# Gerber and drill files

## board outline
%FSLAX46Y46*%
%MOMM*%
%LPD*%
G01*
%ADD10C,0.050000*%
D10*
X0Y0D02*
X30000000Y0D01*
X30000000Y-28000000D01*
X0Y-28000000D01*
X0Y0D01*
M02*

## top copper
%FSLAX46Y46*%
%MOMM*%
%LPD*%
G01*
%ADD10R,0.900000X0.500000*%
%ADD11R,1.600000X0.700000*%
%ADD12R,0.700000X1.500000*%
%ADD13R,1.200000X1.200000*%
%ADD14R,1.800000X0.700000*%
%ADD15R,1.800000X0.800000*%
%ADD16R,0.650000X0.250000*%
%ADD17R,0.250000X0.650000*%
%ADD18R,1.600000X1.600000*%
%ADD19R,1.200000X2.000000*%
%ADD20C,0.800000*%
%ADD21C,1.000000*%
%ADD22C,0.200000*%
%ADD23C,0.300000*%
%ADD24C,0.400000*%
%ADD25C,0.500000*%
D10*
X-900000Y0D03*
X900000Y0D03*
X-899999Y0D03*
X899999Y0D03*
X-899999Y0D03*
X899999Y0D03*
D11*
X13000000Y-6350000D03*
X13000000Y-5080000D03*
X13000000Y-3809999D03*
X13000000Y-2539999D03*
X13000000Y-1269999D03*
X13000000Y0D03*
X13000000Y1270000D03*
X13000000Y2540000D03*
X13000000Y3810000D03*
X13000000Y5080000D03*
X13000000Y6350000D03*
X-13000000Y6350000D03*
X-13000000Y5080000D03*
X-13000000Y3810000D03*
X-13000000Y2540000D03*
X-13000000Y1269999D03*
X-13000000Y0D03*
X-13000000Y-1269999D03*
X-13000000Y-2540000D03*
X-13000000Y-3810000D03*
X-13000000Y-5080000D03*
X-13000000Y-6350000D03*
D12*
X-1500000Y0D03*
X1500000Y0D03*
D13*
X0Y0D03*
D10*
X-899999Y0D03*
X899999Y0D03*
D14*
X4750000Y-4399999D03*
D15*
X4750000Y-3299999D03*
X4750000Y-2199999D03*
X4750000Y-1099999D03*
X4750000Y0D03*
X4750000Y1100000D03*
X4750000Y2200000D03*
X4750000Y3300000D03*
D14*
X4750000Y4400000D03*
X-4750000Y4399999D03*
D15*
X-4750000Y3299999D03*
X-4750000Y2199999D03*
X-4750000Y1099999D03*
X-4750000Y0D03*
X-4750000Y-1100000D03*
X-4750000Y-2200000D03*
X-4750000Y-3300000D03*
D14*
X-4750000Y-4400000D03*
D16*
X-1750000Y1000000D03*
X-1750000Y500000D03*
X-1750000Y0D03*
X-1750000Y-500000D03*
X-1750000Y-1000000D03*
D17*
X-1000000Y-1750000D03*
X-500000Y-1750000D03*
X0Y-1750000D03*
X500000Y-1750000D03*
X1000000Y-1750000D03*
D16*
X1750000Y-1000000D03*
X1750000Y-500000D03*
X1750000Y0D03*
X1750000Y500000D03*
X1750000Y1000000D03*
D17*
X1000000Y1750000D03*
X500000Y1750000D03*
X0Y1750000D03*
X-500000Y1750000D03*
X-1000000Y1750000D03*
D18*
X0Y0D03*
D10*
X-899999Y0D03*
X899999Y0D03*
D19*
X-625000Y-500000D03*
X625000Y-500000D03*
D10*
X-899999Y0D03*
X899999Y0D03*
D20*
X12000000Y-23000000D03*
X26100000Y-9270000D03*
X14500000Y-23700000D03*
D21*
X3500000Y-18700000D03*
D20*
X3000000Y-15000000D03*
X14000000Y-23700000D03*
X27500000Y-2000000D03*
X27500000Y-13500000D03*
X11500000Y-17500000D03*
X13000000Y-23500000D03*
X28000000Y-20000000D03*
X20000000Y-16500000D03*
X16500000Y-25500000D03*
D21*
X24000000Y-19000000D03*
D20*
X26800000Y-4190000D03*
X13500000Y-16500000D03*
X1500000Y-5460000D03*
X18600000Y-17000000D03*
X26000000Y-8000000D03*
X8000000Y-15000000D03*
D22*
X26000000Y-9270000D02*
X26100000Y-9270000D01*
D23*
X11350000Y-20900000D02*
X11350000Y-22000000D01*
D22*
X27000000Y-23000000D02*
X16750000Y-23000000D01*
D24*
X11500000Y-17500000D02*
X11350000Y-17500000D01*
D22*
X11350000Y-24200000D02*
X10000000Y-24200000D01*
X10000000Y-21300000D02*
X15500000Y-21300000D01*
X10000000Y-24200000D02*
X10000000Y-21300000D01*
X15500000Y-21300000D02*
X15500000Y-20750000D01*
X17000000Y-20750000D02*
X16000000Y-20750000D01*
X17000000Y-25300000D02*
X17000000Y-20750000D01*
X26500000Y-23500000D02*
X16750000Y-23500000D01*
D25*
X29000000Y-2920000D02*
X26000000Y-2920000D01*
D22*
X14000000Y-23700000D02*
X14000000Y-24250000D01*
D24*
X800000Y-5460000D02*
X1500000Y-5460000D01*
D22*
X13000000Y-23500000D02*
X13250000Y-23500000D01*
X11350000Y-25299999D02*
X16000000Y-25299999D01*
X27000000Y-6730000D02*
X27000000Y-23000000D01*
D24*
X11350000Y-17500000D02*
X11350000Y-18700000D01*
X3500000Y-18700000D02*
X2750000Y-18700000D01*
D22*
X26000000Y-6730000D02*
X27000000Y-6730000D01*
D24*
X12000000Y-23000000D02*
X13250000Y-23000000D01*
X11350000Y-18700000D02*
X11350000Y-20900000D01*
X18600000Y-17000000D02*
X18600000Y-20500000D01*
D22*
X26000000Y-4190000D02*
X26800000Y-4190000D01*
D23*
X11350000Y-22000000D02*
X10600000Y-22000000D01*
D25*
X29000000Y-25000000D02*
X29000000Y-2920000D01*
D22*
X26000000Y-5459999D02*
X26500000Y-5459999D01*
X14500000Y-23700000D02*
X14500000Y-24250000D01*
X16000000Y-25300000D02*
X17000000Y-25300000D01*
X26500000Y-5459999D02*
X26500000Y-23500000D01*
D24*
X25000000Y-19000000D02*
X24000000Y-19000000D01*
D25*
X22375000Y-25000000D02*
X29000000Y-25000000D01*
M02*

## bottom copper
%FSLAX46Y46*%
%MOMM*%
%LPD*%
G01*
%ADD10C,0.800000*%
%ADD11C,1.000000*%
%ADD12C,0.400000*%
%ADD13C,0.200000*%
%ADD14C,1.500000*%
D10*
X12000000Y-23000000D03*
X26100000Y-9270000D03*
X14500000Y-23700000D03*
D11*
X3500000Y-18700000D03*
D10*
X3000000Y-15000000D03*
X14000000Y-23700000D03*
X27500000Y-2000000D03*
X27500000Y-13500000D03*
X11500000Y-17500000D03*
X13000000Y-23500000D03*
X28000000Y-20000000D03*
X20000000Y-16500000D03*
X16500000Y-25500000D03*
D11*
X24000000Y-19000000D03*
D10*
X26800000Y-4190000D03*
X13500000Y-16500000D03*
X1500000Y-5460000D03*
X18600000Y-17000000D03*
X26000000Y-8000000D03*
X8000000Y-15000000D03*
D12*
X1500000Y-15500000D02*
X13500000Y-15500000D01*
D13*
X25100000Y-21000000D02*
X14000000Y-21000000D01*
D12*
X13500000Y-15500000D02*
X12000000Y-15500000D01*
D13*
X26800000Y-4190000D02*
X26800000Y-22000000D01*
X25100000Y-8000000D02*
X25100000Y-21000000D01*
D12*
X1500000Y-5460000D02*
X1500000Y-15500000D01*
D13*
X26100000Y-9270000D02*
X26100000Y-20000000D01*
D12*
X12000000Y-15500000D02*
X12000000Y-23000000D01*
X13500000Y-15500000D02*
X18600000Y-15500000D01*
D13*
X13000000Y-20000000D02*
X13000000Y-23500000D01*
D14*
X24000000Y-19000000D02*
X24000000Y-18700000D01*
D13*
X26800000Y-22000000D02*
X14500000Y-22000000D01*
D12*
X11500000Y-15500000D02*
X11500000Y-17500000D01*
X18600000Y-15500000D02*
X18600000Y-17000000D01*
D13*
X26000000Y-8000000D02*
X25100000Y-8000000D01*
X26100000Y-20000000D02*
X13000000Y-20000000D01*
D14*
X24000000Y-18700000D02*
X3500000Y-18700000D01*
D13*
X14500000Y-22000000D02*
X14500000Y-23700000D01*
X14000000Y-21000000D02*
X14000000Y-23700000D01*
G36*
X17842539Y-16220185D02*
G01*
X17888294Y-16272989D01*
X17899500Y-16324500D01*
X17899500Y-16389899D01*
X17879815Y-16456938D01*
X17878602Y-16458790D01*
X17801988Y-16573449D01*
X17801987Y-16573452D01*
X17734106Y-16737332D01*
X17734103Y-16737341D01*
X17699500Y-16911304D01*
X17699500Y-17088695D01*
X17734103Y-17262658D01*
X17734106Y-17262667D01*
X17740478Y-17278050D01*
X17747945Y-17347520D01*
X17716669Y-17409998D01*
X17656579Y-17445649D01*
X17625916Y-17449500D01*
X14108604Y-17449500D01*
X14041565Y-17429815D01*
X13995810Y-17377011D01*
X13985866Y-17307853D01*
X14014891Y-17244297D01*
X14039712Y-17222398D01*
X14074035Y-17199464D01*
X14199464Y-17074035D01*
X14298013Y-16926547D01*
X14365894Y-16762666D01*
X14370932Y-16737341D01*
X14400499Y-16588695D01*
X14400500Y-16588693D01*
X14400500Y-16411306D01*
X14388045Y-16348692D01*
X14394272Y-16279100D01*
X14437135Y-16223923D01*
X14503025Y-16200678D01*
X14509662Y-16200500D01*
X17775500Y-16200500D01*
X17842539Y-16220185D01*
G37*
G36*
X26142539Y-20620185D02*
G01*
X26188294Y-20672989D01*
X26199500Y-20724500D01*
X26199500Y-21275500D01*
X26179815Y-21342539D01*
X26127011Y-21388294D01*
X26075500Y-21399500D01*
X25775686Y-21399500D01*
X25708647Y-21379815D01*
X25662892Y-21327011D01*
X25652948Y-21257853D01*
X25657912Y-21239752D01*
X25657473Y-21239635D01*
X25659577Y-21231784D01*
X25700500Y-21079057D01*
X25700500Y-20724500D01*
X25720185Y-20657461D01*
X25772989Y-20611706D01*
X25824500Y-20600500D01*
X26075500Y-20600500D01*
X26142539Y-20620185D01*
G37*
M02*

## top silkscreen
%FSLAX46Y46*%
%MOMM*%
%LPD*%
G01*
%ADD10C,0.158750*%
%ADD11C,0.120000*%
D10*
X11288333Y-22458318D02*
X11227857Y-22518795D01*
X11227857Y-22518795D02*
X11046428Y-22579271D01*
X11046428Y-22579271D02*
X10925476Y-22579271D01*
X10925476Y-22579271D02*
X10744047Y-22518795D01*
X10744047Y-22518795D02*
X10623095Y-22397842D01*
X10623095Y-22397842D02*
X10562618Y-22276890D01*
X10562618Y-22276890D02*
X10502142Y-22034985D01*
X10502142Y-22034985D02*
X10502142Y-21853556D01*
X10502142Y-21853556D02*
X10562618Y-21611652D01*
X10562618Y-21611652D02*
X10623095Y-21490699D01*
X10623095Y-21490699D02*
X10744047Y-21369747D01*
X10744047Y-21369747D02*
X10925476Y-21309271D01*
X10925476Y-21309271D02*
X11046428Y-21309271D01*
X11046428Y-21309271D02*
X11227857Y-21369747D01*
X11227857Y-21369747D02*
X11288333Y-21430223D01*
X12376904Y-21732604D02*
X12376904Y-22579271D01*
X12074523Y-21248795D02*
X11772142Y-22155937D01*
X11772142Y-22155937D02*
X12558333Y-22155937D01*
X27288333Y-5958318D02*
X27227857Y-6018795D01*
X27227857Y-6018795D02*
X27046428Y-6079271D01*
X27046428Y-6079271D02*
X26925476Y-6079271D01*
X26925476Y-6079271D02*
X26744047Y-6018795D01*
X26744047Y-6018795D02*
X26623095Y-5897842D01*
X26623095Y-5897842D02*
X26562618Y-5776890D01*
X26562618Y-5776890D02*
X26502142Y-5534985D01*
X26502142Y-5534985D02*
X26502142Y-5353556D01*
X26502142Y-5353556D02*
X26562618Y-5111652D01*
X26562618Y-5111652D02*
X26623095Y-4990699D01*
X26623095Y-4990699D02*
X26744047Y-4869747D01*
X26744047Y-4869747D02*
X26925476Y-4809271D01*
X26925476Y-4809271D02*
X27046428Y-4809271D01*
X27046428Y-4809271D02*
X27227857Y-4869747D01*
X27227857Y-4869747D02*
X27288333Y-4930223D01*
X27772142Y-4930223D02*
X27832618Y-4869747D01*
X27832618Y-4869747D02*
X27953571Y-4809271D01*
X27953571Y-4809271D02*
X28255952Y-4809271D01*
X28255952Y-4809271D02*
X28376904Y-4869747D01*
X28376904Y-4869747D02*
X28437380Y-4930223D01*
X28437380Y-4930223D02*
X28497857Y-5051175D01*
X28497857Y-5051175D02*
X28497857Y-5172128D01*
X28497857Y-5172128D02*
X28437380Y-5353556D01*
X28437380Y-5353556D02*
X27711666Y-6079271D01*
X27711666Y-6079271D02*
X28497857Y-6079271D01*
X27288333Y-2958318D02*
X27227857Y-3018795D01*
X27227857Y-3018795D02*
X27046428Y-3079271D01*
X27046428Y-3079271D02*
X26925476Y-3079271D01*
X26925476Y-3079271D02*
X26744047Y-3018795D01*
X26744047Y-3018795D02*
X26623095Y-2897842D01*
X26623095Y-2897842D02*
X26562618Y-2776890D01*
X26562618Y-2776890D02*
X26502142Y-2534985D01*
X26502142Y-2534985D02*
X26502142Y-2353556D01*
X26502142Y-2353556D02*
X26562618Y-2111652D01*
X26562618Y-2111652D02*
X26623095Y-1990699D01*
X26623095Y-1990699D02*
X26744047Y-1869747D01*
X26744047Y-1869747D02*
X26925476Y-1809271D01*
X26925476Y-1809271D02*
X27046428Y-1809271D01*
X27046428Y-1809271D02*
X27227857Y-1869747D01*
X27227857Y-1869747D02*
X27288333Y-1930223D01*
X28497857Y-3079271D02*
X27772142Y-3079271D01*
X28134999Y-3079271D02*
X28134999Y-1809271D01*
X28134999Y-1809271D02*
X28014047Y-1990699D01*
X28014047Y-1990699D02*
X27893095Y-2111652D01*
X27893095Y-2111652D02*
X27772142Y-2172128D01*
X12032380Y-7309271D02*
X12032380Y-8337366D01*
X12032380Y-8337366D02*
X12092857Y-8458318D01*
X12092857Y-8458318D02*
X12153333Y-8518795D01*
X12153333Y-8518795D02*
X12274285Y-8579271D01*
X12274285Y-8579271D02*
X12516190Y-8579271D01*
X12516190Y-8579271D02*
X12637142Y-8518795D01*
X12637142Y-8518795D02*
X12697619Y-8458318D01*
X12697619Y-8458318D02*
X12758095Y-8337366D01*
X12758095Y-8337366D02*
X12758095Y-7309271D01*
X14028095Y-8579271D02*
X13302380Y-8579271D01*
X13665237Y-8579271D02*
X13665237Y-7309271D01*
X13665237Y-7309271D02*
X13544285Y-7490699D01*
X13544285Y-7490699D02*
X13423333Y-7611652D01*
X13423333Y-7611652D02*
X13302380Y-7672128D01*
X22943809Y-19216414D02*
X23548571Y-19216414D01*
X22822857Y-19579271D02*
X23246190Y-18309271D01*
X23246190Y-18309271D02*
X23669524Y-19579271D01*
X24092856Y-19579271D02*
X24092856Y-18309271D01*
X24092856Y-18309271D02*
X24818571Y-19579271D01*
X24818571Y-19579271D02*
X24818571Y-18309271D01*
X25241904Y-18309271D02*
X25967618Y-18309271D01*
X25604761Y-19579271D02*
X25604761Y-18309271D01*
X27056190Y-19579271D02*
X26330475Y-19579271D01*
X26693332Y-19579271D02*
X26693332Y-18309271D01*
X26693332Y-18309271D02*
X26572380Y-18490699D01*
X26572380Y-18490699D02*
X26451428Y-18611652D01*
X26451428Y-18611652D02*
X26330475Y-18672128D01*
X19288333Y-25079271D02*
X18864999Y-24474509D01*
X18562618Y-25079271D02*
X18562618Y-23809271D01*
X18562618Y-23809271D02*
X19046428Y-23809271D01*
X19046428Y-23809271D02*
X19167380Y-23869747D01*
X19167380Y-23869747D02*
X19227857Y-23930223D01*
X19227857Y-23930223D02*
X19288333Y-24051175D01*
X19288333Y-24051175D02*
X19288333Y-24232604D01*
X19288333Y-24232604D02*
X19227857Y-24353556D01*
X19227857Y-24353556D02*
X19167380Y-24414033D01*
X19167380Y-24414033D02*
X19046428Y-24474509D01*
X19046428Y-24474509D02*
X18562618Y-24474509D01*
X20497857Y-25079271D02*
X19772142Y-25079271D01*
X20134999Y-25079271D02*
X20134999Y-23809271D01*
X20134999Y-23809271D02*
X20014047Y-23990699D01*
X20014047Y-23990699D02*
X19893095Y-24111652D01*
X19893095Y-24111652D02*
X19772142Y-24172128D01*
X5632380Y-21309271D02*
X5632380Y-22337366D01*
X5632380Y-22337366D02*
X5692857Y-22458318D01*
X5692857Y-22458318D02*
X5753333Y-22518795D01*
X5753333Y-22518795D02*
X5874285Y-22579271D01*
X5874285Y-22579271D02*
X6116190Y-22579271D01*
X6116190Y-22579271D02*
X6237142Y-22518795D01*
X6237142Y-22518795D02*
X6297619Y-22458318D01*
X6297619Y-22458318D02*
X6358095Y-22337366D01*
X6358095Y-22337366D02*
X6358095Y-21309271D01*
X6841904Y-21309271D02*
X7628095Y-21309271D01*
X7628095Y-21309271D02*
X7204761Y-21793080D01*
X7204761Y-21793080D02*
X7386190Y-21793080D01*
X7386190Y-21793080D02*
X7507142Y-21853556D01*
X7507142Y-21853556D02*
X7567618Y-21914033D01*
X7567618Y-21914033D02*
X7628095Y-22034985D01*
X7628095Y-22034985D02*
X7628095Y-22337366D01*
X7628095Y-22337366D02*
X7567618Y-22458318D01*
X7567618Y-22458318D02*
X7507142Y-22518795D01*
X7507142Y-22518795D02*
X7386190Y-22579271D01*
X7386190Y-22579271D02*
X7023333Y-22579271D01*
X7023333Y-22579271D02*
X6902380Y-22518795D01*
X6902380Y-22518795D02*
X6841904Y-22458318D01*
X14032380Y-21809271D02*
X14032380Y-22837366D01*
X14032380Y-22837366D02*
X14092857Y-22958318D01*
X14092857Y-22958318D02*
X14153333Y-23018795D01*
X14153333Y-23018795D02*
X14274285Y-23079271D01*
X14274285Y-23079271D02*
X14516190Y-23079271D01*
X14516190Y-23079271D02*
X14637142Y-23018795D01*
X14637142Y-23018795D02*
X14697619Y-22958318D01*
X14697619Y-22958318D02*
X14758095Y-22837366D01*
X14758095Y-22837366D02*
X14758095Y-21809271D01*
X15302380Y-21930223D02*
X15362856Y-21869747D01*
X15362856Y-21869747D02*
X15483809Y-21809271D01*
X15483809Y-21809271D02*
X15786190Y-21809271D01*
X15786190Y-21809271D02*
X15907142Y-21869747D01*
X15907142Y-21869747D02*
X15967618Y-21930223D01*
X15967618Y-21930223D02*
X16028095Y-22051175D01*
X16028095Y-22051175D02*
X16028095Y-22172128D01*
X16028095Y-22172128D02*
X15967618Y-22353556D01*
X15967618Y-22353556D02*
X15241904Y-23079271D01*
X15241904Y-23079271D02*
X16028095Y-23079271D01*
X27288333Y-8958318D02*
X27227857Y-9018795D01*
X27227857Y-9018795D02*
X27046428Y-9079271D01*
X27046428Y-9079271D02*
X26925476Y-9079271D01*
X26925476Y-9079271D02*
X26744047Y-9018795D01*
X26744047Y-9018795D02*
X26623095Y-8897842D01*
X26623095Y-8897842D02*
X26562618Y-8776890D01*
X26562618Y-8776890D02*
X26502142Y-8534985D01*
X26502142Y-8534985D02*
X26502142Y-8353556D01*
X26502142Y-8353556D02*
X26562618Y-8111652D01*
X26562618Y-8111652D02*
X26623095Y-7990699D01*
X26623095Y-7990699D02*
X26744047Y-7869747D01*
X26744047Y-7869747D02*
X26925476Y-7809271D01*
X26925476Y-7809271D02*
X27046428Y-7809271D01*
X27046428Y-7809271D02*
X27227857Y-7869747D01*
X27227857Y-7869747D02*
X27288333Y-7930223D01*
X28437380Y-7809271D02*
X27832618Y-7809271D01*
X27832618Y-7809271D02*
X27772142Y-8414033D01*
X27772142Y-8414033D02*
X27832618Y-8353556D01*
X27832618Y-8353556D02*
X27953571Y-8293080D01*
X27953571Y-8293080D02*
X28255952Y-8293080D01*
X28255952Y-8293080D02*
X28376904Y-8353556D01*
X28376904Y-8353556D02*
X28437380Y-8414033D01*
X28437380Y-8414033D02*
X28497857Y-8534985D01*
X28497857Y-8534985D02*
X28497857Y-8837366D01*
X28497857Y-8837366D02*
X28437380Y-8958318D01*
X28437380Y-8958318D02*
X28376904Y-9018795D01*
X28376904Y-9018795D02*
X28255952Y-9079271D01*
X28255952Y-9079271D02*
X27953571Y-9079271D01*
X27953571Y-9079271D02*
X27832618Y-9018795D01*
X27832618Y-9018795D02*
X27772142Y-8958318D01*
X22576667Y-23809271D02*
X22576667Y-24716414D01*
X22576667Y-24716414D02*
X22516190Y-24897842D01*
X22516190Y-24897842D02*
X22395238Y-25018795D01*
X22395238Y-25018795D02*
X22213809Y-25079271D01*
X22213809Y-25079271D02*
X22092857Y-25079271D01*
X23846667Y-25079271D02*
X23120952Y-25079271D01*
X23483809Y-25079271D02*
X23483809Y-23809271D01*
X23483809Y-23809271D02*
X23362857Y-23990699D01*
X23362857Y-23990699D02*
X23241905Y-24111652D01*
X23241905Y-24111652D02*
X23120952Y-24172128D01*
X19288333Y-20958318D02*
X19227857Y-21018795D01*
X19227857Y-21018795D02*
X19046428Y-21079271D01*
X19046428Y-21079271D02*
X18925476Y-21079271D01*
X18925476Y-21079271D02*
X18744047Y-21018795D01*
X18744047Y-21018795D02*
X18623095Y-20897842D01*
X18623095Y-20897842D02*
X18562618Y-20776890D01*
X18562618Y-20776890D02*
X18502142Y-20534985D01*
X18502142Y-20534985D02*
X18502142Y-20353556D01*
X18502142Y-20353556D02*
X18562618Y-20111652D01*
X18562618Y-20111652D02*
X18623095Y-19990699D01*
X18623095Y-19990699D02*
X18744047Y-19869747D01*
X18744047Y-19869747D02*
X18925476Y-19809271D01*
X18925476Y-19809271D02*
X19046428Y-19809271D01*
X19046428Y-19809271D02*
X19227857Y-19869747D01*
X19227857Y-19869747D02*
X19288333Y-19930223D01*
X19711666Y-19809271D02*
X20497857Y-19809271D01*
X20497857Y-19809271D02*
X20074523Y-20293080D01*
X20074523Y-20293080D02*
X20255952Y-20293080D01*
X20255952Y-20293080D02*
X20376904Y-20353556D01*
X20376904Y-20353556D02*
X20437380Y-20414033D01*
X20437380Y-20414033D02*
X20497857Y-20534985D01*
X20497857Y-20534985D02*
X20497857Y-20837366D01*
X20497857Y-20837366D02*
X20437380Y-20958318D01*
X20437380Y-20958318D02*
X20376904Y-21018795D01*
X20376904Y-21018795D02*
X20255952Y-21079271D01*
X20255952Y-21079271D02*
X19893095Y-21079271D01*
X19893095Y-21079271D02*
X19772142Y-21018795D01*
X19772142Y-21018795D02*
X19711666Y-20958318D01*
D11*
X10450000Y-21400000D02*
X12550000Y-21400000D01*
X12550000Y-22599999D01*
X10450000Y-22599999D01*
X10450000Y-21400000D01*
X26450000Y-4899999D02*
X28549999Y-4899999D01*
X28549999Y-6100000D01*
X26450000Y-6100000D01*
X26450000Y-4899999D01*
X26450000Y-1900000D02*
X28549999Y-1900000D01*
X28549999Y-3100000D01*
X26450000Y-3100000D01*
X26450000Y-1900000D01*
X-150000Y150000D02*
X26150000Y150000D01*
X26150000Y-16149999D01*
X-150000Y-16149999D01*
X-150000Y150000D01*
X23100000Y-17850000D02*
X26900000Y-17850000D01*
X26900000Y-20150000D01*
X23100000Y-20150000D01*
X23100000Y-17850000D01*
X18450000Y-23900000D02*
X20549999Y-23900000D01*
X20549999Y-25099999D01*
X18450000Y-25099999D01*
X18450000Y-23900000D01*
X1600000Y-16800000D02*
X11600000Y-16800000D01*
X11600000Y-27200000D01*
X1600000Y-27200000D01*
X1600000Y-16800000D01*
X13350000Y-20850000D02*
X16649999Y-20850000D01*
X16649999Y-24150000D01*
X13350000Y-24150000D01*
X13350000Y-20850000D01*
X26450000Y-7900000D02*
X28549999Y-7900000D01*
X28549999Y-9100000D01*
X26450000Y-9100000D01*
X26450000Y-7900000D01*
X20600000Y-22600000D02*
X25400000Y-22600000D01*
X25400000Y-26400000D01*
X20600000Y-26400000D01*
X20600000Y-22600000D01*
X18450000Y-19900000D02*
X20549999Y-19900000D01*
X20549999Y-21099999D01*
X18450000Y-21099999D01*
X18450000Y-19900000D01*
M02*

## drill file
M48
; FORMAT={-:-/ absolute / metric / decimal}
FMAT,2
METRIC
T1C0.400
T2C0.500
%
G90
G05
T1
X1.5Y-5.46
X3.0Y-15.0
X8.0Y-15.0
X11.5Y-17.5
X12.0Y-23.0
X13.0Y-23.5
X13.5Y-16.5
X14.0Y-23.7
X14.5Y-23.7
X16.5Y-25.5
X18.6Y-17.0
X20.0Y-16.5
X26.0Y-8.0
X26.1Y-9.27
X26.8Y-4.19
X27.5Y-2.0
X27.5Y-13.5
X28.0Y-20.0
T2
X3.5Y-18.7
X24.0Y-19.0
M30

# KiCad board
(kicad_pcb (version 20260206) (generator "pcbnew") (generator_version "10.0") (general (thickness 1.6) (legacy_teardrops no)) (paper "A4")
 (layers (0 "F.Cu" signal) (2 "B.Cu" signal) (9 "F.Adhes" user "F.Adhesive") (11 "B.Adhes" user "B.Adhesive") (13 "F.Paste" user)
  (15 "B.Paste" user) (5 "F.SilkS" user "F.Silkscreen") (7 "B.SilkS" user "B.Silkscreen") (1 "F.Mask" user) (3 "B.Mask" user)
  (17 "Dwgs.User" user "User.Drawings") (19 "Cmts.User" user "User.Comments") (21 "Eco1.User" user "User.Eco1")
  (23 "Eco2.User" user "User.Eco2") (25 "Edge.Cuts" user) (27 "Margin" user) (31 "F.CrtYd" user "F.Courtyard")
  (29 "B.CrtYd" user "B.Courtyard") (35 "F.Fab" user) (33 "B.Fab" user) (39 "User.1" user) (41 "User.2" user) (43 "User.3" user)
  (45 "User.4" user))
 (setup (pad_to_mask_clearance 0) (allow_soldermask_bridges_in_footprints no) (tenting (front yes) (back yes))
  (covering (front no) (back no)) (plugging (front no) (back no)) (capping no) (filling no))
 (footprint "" (layer "F.Cu") (at 11.5 22)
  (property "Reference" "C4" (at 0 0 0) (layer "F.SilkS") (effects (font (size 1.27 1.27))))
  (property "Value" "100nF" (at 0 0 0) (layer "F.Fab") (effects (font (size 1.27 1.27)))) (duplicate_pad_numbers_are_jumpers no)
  (fp_rect (start -1.05 -0.6) (end 1.05 0.599999) (stroke (width 0.12) (type default)) (fill no) (layer "F.SilkS"))
  (pad "1" smd rect (at -12.4 -22) (size 0.9 0.5) (layers "F.Cu" "F.Mask" "F.Paste") (thermal_bridge_angle 45))
  (pad "2" smd rect (at -10.6 -22) (size 0.9 0.5) (layers "F.Cu" "F.Mask" "F.Paste") (thermal_bridge_angle 45)))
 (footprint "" (layer "F.Cu") (at 27.5 5.5)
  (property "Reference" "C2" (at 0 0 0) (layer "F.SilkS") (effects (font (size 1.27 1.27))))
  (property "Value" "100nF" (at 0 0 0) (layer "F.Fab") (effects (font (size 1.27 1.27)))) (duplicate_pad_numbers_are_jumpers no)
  (fp_rect (start -1.05 -0.600001) (end 1.049999 0.6) (stroke (width 0.12) (type default)) (fill no) (layer "F.SilkS"))
  (pad "1" smd rect (at -28.399999 -5.5) (size 0.9 0.5) (layers "F.Cu" "F.Mask" "F.Paste") (thermal_bridge_angle 45))
  (pad "2" smd rect (at -26.600001 -5.5) (size 0.9 0.5) (layers "F.Cu" "F.Mask" "F.Paste") (thermal_bridge_angle 45)))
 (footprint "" (layer "F.Cu") (at 27.5 2.5)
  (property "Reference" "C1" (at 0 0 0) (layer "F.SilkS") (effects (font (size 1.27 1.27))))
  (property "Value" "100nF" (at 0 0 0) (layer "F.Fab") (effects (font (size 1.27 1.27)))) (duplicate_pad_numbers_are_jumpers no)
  (fp_rect (start -1.05 -0.6) (end 1.049999 0.6) (stroke (width 0.12) (type default)) (fill no) (layer "F.SilkS"))
  (pad "1" smd rect (at -28.399999 -2.5) (size 0.9 0.5) (layers "F.Cu" "F.Mask" "F.Paste") (thermal_bridge_angle 45))
  (pad "2" smd rect (at -26.600001 -2.5) (size 0.9 0.5) (layers "F.Cu" "F.Mask" "F.Paste") (thermal_bridge_angle 45)))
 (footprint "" (layer "F.Cu") (at 13 8)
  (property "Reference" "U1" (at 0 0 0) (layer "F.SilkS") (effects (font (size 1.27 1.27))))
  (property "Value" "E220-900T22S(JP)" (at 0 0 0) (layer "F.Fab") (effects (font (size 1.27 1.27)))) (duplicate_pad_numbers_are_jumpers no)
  (fp_rect (start -13.15 -8.15) (end 13.15 8.149999) (stroke (width 0.12) (type default)) (fill no) (layer "F.SilkS"))
  (pad "1" smd rect (at 0 -1.65) (size 1.6 0.7) (layers "F.Cu" "F.Mask" "F.Paste") (thermal_bridge_angle 45))
  (pad "2" smd rect (at 0 -2.92) (size 1.6 0.7) (layers "F.Cu" "F.Mask" "F.Paste") (thermal_bridge_angle 45))
  (pad "3" smd rect (at 0 -4.190001) (size 1.6 0.7) (layers "F.Cu" "F.Mask" "F.Paste") (thermal_bridge_angle 45))
  (pad "4" smd rect (at 0 -5.460001) (size 1.6 0.7) (layers "F.Cu" "F.Mask" "F.Paste") (thermal_bridge_angle 45))
  (pad "5" smd rect (at 0 -6.730001) (size 1.6 0.7) (layers "F.Cu" "F.Mask" "F.Paste") (thermal_bridge_angle 45))
  (pad "6" smd rect (at 0 -8) (size 1.6 0.7) (layers "F.Cu" "F.Mask" "F.Paste") (thermal_bridge_angle 45))
  (pad "7" smd rect (at 0 -9.27) (size 1.6 0.7) (layers "F.Cu" "F.Mask" "F.Paste") (thermal_bridge_angle 45))
  (pad "8" smd rect (at 0 -10.54) (size 1.6 0.7) (layers "F.Cu" "F.Mask" "F.Paste") (thermal_bridge_angle 45))
  (pad "9" smd rect (at 0 -11.81) (size 1.6 0.7) (layers "F.Cu" "F.Mask" "F.Paste") (thermal_bridge_angle 45))
  (pad "10" smd rect (at 0 -13.08) (size 1.6 0.7) (layers "F.Cu" "F.Mask" "F.Paste") (thermal_bridge_angle 45))
  (pad "11" smd rect (at 0 -14.35) (size 1.6 0.7) (layers "F.Cu" "F.Mask" "F.Paste") (thermal_bridge_angle 45))
  (pad "12" smd rect (at -26 -14.35) (size 1.6 0.7) (layers "F.Cu" "F.Mask" "F.Paste") (thermal_bridge_angle 45))
  (pad "13" smd rect (at -26 -13.08) (size 1.6 0.7) (layers "F.Cu" "F.Mask" "F.Paste") (thermal_bridge_angle 45))
  (pad "14" smd rect (at -26 -11.81) (size 1.6 0.7) (layers "F.Cu" "F.Mask" "F.Paste") (thermal_bridge_angle 45))
  (pad "15" smd rect (at -26 -10.54) (size 1.6 0.7) (layers "F.Cu" "F.Mask" "F.Paste") (thermal_bridge_angle 45))
  (pad "16" smd rect (at -26 -9.269999) (size 1.6 0.7) (layers "F.Cu" "F.Mask" "F.Paste") (thermal_bridge_angle 45))
  (pad "17" smd rect (at -26 -8) (size 1.6 0.7) (layers "F.Cu" "F.Mask" "F.Paste") (thermal_bridge_angle 45))
  (pad "18" smd rect (at -26 -6.730001) (size 1.6 0.7) (layers "F.Cu" "F.Mask" "F.Paste") (thermal_bridge_angle 45))
  (pad "19" smd rect (at -26 -5.46) (size 1.6 0.7) (layers "F.Cu" "F.Mask" "F.Paste") (thermal_bridge_angle 45))
  (pad "20" smd rect (at -26 -4.19) (size 1.6 0.7) (layers "F.Cu" "F.Mask" "F.Paste") (thermal_bridge_angle 45))
  (pad "21" smd rect (at -26 -2.92) (size 1.6 0.7) (layers "F.Cu" "F.Mask" "F.Paste") (thermal_bridge_angle 45))
  (pad "22" smd rect (at -26 -1.65) (size 1.6 0.7) (layers "F.Cu" "F.Mask" "F.Paste") (thermal_bridge_angle 45)))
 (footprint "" (layer "F.Cu") (at 25 19)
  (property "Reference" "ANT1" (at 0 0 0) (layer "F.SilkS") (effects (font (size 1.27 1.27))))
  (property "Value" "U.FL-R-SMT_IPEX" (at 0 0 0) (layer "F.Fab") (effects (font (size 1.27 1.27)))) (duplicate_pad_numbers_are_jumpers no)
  (fp_rect (start -1.9 -1.15) (end 1.9 1.15) (stroke (width 0.12) (type default)) (fill no) (layer "F.SilkS"))
  (pad "G1" smd rect (at -26.5 -19) (size 0.7 1.5) (layers "F.Cu" "F.Mask" "F.Paste") (thermal_bridge_angle 45))
  (pad "G2" smd rect (at -23.5 -19) (size 0.7 1.5) (layers "F.Cu" "F.Mask" "F.Paste") (thermal_bridge_angle 45))
  (pad "S" smd rect (at -25 -19) (size 1.2 1.2) (layers "F.Cu" "F.Mask" "F.Paste") (thermal_bridge_angle 45)))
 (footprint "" (layer "F.Cu") (at 19.5 24.5)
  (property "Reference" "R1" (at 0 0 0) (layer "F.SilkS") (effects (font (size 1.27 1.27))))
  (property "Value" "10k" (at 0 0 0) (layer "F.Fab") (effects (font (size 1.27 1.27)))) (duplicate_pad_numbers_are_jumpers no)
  (fp_rect (start -1.05 -0.6) (end 1.049999 0.599999) (stroke (width 0.12) (type default)) (fill no) (layer "F.SilkS"))
  (pad "1" smd rect (at -20.399999 -24.5) (size 0.9 0.5) (layers "F.Cu" "F.Mask" "F.Paste") (thermal_bridge_angle 45))
  (pad "2" smd rect (at -18.600001 -24.5) (size 0.9 0.5) (layers "F.Cu" "F.Mask" "F.Paste") (thermal_bridge_angle 45)))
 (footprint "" (layer "F.Cu") (at 6.6 22)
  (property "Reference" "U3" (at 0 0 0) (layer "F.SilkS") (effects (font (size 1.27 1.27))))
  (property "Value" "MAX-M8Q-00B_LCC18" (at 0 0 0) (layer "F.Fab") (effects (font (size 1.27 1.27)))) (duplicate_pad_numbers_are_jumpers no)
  (fp_rect (start -5 -5.2) (end 5 5.2) (stroke (width 0.12) (type default)) (fill no) (layer "F.SilkS"))
  (pad "1" smd rect (at -1.85 -17.600001) (size 1.8 0.7) (layers "F.Cu" "F.Mask" "F.Paste") (thermal_bridge_angle 45))
  (pad "2" smd rect (at -1.85 -18.700001) (size 1.8 0.8) (layers "F.Cu" "F.Mask" "F.Paste") (thermal_bridge_angle 45))
  (pad "3" smd rect (at -1.85 -19.800001) (size 1.8 0.8) (layers "F.Cu" "F.Mask" "F.Paste") (thermal_bridge_angle 45))
  (pad "4" smd rect (at -1.85 -20.900001) (size 1.8 0.8) (layers "F.Cu" "F.Mask" "F.Paste") (thermal_bridge_angle 45))
  (pad "5" smd rect (at -1.85 -22) (size 1.8 0.8) (layers "F.Cu" "F.Mask" "F.Paste") (thermal_bridge_angle 45))
  (pad "6" smd rect (at -1.85 -23.1) (size 1.8 0.8) (layers "F.Cu" "F.Mask" "F.Paste") (thermal_bridge_angle 45))
  (pad "7" smd rect (at -1.85 -24.2) (size 1.8 0.8) (layers "F.Cu" "F.Mask" "F.Paste") (thermal_bridge_angle 45))
  (pad "8" smd rect (at -1.85 -25.3) (size 1.8 0.8) (layers "F.Cu" "F.Mask" "F.Paste") (thermal_bridge_angle 45))
  (pad "9" smd rect (at -1.85 -26.4) (size 1.8 0.7) (layers "F.Cu" "F.Mask" "F.Paste") (thermal_bridge_angle 45))
  (pad "10" smd rect (at -11.35 -26.399999) (size 1.8 0.7) (layers "F.Cu" "F.Mask" "F.Paste") (thermal_bridge_angle 45))
  (pad "11" smd rect (at -11.35 -25.299999) (size 1.8 0.8) (layers "F.Cu" "F.Mask" "F.Paste") (thermal_bridge_angle 45))
  (pad "12" smd rect (at -11.35 -24.199999) (size 1.8 0.8) (layers "F.Cu" "F.Mask" "F.Paste") (thermal_bridge_angle 45))
  (pad "13" smd rect (at -11.35 -23.099999) (size 1.8 0.8) (layers "F.Cu" "F.Mask" "F.Paste") (thermal_bridge_angle 45))
  (pad "14" smd rect (at -11.35 -22) (size 1.8 0.8) (layers "F.Cu" "F.Mask" "F.Paste") (thermal_bridge_angle 45))
  (pad "15" smd rect (at -11.35 -20.9) (size 1.8 0.8) (layers "F.Cu" "F.Mask" "F.Paste") (thermal_bridge_angle 45))
  (pad "16" smd rect (at -11.35 -19.8) (size 1.8 0.8) (layers "F.Cu" "F.Mask" "F.Paste") (thermal_bridge_angle 45))
  (pad "17" smd rect (at -11.35 -18.7) (size 1.8 0.8) (layers "F.Cu" "F.Mask" "F.Paste") (thermal_bridge_angle 45))
  (pad "18" smd rect (at -11.35 -17.6) (size 1.8 0.7) (layers "F.Cu" "F.Mask" "F.Paste") (thermal_bridge_angle 45)))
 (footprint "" (layer "F.Cu") (at 15 22.5)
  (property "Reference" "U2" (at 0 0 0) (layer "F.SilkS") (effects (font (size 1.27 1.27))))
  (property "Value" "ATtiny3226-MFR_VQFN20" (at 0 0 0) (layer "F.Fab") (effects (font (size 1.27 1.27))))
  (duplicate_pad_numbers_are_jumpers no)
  (fp_rect (start -1.65 -1.65) (end 1.649999 1.65) (stroke (width 0.12) (type default)) (fill no) (layer "F.SilkS"))
  (pad "1" smd rect (at -16.75 -23.5) (size 0.65 0.25) (layers "F.Cu" "F.Mask" "F.Paste") (thermal_bridge_angle 45))
  (pad "2" smd rect (at -16.75 -23) (size 0.65 0.25) (layers "F.Cu" "F.Mask" "F.Paste") (thermal_bridge_angle 45))
  (pad "3" smd rect (at -16.75 -22.5) (size 0.65 0.25) (layers "F.Cu" "F.Mask" "F.Paste") (thermal_bridge_angle 45))
  (pad "4" smd rect (at -16.75 -22) (size 0.65 0.25) (layers "F.Cu" "F.Mask" "F.Paste") (thermal_bridge_angle 45))
  (pad "5" smd rect (at -16.75 -21.5) (size 0.65 0.25) (layers "F.Cu" "F.Mask" "F.Paste") (thermal_bridge_angle 45))
  (pad "6" smd rect (at -16 -20.75) (size 0.25 0.65) (layers "F.Cu" "F.Mask" "F.Paste") (thermal_bridge_angle 45))
  (pad "7" smd rect (at -15.5 -20.75) (size 0.25 0.65) (layers "F.Cu" "F.Mask" "F.Paste") (thermal_bridge_angle 45))
  (pad "8" smd rect (at -15 -20.75) (size 0.25 0.65) (layers "F.Cu" "F.Mask" "F.Paste") (thermal_bridge_angle 45))
  (pad "9" smd rect (at -14.5 -20.75) (size 0.25 0.65) (layers "F.Cu" "F.Mask" "F.Paste") (thermal_bridge_angle 45))
  (pad "10" smd rect (at -14 -20.75) (size 0.25 0.65) (layers "F.Cu" "F.Mask" "F.Paste") (thermal_bridge_angle 45))
  (pad "11" smd rect (at -13.25 -21.5) (size 0.65 0.25) (layers "F.Cu" "F.Mask" "F.Paste") (thermal_bridge_angle 45))
  (pad "12" smd rect (at -13.25 -22) (size 0.65 0.25) (layers "F.Cu" "F.Mask" "F.Paste") (thermal_bridge_angle 45))
  (pad "13" smd rect (at -13.25 -22.5) (size 0.65 0.25) (layers "F.Cu" "F.Mask" "F.Paste") (thermal_bridge_angle 45))
  (pad "14" smd rect (at -13.25 -23) (size 0.65 0.25) (layers "F.Cu" "F.Mask" "F.Paste") (thermal_bridge_angle 45))
  (pad "15" smd rect (at -13.25 -23.5) (size 0.65 0.25) (layers "F.Cu" "F.Mask" "F.Paste") (thermal_bridge_angle 45))
  (pad "16" smd rect (at -14 -24.25) (size 0.25 0.65) (layers "F.Cu" "F.Mask" "F.Paste") (thermal_bridge_angle 45))
  (pad "17" smd rect (at -14.5 -24.25) (size 0.25 0.65) (layers "F.Cu" "F.Mask" "F.Paste") (thermal_bridge_angle 45))
  (pad "18" smd rect (at -15 -24.25) (size 0.25 0.65) (layers "F.Cu" "F.Mask" "F.Paste") (thermal_bridge_angle 45))
  (pad "19" smd rect (at -15.5 -24.25) (size 0.25 0.65) (layers "F.Cu" "F.Mask" "F.Paste") (thermal_bridge_angle 45))
  (pad "20" smd rect (at -16 -24.25) (size 0.25 0.65) (layers "F.Cu" "F.Mask" "F.Paste") (thermal_bridge_angle 45))
  (pad "EP" smd rect (at -15 -22.5) (size 1.6 1.6) (layers "F.Cu" "F.Mask" "F.Paste") (thermal_bridge_angle 45)))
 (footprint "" (layer "F.Cu") (at 27.5 8.5)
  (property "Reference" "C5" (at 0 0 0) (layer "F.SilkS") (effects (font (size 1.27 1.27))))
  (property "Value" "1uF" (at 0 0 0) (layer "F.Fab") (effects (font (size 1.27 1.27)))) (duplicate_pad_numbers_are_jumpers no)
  (fp_rect (start -1.05 -0.6) (end 1.049999 0.6) (stroke (width 0.12) (type default)) (fill no) (layer "F.SilkS"))
  (pad "1" smd rect (at -28.399999 -8.5) (size 0.9 0.5) (layers "F.Cu" "F.Mask" "F.Paste") (thermal_bridge_angle 45))
  (pad "2" smd rect (at -26.600001 -8.5) (size 0.9 0.5) (layers "F.Cu" "F.Mask" "F.Paste") (thermal_bridge_angle 45)))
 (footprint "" (layer "F.Cu") (at 23 24.5)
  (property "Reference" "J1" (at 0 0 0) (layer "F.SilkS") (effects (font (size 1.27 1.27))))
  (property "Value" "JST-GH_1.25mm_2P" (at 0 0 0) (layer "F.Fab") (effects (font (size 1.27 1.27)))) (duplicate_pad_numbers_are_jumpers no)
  (fp_rect (start -2.4 -1.9) (end 2.4 1.9) (stroke (width 0.12) (type default)) (fill no) (layer "F.SilkS"))
  (pad "1" smd rect (at -23.625 -24) (size 1.2 2) (layers "F.Cu" "F.Mask" "F.Paste") (thermal_bridge_angle 45))
  (pad "2" smd rect (at -22.375 -24) (size 1.2 2) (layers "F.Cu" "F.Mask" "F.Paste") (thermal_bridge_angle 45)))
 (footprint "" (layer "F.Cu") (at 19.5 20.5)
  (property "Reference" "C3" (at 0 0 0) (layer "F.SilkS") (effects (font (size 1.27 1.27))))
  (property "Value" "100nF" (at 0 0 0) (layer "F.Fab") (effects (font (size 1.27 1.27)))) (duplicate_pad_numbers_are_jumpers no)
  (fp_rect (start -1.05 -0.6) (end 1.049999 0.599999) (stroke (width 0.12) (type default)) (fill no) (layer "F.SilkS"))
  (pad "1" smd rect (at -20.399999 -20.5) (size 0.9 0.5) (layers "F.Cu" "F.Mask" "F.Paste") (thermal_bridge_angle 45))
  (pad "2" smd rect (at -18.600001 -20.5) (size 0.9 0.5) (layers "F.Cu" "F.Mask" "F.Paste") (thermal_bridge_angle 45)))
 (gr_rect (start 0 0) (end 30 28) (stroke (width 0.05) (type default)) (fill no) (layer "Edge.Cuts"))
 (segment (start 26 9.27) (end 26.1 9.27) (width 0.2) (layer "F.Cu") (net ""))
 (segment (start 11.35 20.9) (end 11.35 22) (width 0.3) (layer "F.Cu") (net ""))
 (segment (start 27 23) (end 16.75 23) (width 0.2) (layer "F.Cu") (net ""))
 (segment (start 11.5 17.5) (end 11.35 17.5) (width 0.4) (layer "F.Cu") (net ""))
 (segment (start 11.35 24.2) (end 10 24.2) (width 0.2) (layer "F.Cu") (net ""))
 (segment (start 10 21.3) (end 15.5 21.3) (width 0.2) (layer "F.Cu") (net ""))
 (segment (start 10 24.2) (end 10 21.3) (width 0.2) (layer "F.Cu") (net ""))
 (segment (start 15.5 21.3) (end 15.5 20.75) (width 0.2) (layer "F.Cu") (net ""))
 (segment (start 17 20.75) (end 16 20.75) (width 0.2) (layer "F.Cu") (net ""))
 (segment (start 17 25.3) (end 17 20.75) (width 0.2) (layer "F.Cu") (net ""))
 (segment (start 26.5 23.5) (end 16.75 23.5) (width 0.2) (layer "F.Cu") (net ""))
 (segment (start 29 2.92) (end 26 2.92) (width 0.5) (layer "F.Cu") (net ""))
 (segment (start 14 23.7) (end 14 24.25) (width 0.2) (layer "F.Cu") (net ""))
 (segment (start 0.8 5.46) (end 1.5 5.46) (width 0.4) (layer "F.Cu") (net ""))
 (segment (start 13 23.5) (end 13.25 23.5) (width 0.2) (layer "F.Cu") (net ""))
 (segment (start 11.35 25.299999) (end 16 25.299999) (width 0.2) (layer "F.Cu") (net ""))
 (segment (start 27 6.73) (end 27 23) (width 0.2) (layer "F.Cu") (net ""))
 (segment (start 11.35 17.5) (end 11.35 18.7) (width 0.4) (layer "F.Cu") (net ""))
 (segment (start 3.5 18.7) (end 2.75 18.7) (width 0.4) (layer "F.Cu") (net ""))
 (segment (start 26 6.73) (end 27 6.73) (width 0.2) (layer "F.Cu") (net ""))
 (segment (start 12 23) (end 13.25 23) (width 0.4) (layer "F.Cu") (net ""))
 (segment (start 11.35 18.7) (end 11.35 20.9) (width 0.4) (layer "F.Cu") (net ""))
 (segment (start 18.6 17) (end 18.6 20.5) (width 0.4) (layer "F.Cu") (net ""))
 (segment (start 26 4.19) (end 26.8 4.19) (width 0.2) (layer "F.Cu") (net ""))
 (segment (start 11.35 22) (end 10.6 22) (width 0.3) (layer "F.Cu") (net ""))
 (segment (start 29 25) (end 29 2.92) (width 0.5) (layer "F.Cu") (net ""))
 (segment (start 26 5.459999) (end 26.5 5.459999) (width 0.2) (layer "F.Cu") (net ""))
 (segment (start 14.5 23.7) (end 14.5 24.25) (width 0.2) (layer "F.Cu") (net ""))
 (segment (start 16 25.3) (end 17 25.3) (width 0.2) (layer "F.Cu") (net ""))
 (segment (start 26.5 5.459999) (end 26.5 23.5) (width 0.2) (layer "F.Cu") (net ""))
 (segment (start 25 19) (end 24 19) (width 0.4) (layer "F.Cu") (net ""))
 (segment (start 22.375 25) (end 29 25) (width 0.5) (layer "F.Cu") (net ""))
 (via (at 12 23) (size 0.8) (drill 0.4) (layers "F.Cu" "B.Cu") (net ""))
 (via (at 26.1 9.27) (size 0.8) (drill 0.4) (layers "F.Cu" "B.Cu") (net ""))
 (via (at 14.5 23.7) (size 0.8) (drill 0.4) (layers "F.Cu" "B.Cu") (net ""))
 (via (at 3.5 18.7) (size 1) (drill 0.5) (layers "F.Cu" "B.Cu") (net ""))
 (via (at 3 15) (size 0.8) (drill 0.4) (layers "F.Cu" "B.Cu") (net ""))
 (via (at 14 23.7) (size 0.8) (drill 0.4) (layers "F.Cu" "B.Cu") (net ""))
 (via (at 27.5 2) (size 0.8) (drill 0.4) (layers "F.Cu" "B.Cu") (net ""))
 (via (at 27.5 13.5) (size 0.8) (drill 0.4) (layers "F.Cu" "B.Cu") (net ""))
 (via (at 11.5 17.5) (size 0.8) (drill 0.4) (layers "F.Cu" "B.Cu") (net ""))
 (via (at 13 23.5) (size 0.8) (drill 0.4) (layers "F.Cu" "B.Cu") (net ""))
 (via (at 28 20) (size 0.8) (drill 0.4) (layers "F.Cu" "B.Cu") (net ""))
 (via (at 20 16.5) (size 0.8) (drill 0.4) (layers "F.Cu" "B.Cu") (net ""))
 (via (at 16.5 25.5) (size 0.8) (drill 0.4) (layers "F.Cu" "B.Cu") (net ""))
 (via (at 24 19) (size 1) (drill 0.5) (layers "F.Cu" "B.Cu") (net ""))
 (via (at 26.8 4.19) (size 0.8) (drill 0.4) (layers "F.Cu" "B.Cu") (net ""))
 (via (at 13.5 16.5) (size 0.8) (drill 0.4) (layers "F.Cu" "B.Cu") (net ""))
 (via (at 1.5 5.46) (size 0.8) (drill 0.4) (layers "F.Cu" "B.Cu") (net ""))
 (via (at 18.6 17) (size 0.8) (drill 0.4) (layers "F.Cu" "B.Cu") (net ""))
 (via (at 26 8) (size 0.8) (drill 0.4) (layers "F.Cu" "B.Cu") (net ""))
 (via (at 8 15) (size 0.8) (drill 0.4) (layers "F.Cu" "B.Cu") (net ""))
 (segment (start 1.5 15.5) (end 13.5 15.5) (width 0.4) (layer "B.Cu") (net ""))
 (segment (start 25.1 21) (end 14 21) (width 0.2) (layer "B.Cu") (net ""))
 (segment (start 13.5 15.5) (end 12 15.5) (width 0.4) (layer "B.Cu") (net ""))
 (segment (start 26.8 4.19) (end 26.8 22) (width 0.2) (layer "B.Cu") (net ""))
 (segment (start 25.1 8) (end 25.1 21) (width 0.2) (layer "B.Cu") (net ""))
 (segment (start 1.5 5.46) (end 1.5 15.5) (width 0.4) (layer "B.Cu") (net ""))
 (segment (start 26.1 9.27) (end 26.1 20) (width 0.2) (layer "B.Cu") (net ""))
 (segment (start 12 15.5) (end 12 23) (width 0.4) (layer "B.Cu") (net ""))
 (segment (start 13.5 15.5) (end 18.6 15.5) (width 0.4) (layer "B.Cu") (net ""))
 (segment (start 13 20) (end 13 23.5) (width 0.2) (layer "B.Cu") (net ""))
 (segment (start 24 19) (end 24 18.7) (width 1.5) (layer "B.Cu") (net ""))
 (segment (start 26.8 22) (end 14.5 22) (width 0.2) (layer "B.Cu") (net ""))
 (segment (start 11.5 15.5) (end 11.5 17.5) (width 0.4) (layer "B.Cu") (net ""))
 (segment (start 18.6 15.5) (end 18.6 17) (width 0.4) (layer "B.Cu") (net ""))
 (segment (start 26 8) (end 25.1 8) (width 0.2) (layer "B.Cu") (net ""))
 (segment (start 26.1 20) (end 13 20) (width 0.2) (layer "B.Cu") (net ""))
 (segment (start 24 18.7) (end 3.5 18.7) (width 1.5) (layer "B.Cu") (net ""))
 (segment (start 14.5 22) (end 14.5 23.7) (width 0.2) (layer "B.Cu") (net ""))
 (segment (start 14 21) (end 14 23.7) (width 0.2) (layer "B.Cu") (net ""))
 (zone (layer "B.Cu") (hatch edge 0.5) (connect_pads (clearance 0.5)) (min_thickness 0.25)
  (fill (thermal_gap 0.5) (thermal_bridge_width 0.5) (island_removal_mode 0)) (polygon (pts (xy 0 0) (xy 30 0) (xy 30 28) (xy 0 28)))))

